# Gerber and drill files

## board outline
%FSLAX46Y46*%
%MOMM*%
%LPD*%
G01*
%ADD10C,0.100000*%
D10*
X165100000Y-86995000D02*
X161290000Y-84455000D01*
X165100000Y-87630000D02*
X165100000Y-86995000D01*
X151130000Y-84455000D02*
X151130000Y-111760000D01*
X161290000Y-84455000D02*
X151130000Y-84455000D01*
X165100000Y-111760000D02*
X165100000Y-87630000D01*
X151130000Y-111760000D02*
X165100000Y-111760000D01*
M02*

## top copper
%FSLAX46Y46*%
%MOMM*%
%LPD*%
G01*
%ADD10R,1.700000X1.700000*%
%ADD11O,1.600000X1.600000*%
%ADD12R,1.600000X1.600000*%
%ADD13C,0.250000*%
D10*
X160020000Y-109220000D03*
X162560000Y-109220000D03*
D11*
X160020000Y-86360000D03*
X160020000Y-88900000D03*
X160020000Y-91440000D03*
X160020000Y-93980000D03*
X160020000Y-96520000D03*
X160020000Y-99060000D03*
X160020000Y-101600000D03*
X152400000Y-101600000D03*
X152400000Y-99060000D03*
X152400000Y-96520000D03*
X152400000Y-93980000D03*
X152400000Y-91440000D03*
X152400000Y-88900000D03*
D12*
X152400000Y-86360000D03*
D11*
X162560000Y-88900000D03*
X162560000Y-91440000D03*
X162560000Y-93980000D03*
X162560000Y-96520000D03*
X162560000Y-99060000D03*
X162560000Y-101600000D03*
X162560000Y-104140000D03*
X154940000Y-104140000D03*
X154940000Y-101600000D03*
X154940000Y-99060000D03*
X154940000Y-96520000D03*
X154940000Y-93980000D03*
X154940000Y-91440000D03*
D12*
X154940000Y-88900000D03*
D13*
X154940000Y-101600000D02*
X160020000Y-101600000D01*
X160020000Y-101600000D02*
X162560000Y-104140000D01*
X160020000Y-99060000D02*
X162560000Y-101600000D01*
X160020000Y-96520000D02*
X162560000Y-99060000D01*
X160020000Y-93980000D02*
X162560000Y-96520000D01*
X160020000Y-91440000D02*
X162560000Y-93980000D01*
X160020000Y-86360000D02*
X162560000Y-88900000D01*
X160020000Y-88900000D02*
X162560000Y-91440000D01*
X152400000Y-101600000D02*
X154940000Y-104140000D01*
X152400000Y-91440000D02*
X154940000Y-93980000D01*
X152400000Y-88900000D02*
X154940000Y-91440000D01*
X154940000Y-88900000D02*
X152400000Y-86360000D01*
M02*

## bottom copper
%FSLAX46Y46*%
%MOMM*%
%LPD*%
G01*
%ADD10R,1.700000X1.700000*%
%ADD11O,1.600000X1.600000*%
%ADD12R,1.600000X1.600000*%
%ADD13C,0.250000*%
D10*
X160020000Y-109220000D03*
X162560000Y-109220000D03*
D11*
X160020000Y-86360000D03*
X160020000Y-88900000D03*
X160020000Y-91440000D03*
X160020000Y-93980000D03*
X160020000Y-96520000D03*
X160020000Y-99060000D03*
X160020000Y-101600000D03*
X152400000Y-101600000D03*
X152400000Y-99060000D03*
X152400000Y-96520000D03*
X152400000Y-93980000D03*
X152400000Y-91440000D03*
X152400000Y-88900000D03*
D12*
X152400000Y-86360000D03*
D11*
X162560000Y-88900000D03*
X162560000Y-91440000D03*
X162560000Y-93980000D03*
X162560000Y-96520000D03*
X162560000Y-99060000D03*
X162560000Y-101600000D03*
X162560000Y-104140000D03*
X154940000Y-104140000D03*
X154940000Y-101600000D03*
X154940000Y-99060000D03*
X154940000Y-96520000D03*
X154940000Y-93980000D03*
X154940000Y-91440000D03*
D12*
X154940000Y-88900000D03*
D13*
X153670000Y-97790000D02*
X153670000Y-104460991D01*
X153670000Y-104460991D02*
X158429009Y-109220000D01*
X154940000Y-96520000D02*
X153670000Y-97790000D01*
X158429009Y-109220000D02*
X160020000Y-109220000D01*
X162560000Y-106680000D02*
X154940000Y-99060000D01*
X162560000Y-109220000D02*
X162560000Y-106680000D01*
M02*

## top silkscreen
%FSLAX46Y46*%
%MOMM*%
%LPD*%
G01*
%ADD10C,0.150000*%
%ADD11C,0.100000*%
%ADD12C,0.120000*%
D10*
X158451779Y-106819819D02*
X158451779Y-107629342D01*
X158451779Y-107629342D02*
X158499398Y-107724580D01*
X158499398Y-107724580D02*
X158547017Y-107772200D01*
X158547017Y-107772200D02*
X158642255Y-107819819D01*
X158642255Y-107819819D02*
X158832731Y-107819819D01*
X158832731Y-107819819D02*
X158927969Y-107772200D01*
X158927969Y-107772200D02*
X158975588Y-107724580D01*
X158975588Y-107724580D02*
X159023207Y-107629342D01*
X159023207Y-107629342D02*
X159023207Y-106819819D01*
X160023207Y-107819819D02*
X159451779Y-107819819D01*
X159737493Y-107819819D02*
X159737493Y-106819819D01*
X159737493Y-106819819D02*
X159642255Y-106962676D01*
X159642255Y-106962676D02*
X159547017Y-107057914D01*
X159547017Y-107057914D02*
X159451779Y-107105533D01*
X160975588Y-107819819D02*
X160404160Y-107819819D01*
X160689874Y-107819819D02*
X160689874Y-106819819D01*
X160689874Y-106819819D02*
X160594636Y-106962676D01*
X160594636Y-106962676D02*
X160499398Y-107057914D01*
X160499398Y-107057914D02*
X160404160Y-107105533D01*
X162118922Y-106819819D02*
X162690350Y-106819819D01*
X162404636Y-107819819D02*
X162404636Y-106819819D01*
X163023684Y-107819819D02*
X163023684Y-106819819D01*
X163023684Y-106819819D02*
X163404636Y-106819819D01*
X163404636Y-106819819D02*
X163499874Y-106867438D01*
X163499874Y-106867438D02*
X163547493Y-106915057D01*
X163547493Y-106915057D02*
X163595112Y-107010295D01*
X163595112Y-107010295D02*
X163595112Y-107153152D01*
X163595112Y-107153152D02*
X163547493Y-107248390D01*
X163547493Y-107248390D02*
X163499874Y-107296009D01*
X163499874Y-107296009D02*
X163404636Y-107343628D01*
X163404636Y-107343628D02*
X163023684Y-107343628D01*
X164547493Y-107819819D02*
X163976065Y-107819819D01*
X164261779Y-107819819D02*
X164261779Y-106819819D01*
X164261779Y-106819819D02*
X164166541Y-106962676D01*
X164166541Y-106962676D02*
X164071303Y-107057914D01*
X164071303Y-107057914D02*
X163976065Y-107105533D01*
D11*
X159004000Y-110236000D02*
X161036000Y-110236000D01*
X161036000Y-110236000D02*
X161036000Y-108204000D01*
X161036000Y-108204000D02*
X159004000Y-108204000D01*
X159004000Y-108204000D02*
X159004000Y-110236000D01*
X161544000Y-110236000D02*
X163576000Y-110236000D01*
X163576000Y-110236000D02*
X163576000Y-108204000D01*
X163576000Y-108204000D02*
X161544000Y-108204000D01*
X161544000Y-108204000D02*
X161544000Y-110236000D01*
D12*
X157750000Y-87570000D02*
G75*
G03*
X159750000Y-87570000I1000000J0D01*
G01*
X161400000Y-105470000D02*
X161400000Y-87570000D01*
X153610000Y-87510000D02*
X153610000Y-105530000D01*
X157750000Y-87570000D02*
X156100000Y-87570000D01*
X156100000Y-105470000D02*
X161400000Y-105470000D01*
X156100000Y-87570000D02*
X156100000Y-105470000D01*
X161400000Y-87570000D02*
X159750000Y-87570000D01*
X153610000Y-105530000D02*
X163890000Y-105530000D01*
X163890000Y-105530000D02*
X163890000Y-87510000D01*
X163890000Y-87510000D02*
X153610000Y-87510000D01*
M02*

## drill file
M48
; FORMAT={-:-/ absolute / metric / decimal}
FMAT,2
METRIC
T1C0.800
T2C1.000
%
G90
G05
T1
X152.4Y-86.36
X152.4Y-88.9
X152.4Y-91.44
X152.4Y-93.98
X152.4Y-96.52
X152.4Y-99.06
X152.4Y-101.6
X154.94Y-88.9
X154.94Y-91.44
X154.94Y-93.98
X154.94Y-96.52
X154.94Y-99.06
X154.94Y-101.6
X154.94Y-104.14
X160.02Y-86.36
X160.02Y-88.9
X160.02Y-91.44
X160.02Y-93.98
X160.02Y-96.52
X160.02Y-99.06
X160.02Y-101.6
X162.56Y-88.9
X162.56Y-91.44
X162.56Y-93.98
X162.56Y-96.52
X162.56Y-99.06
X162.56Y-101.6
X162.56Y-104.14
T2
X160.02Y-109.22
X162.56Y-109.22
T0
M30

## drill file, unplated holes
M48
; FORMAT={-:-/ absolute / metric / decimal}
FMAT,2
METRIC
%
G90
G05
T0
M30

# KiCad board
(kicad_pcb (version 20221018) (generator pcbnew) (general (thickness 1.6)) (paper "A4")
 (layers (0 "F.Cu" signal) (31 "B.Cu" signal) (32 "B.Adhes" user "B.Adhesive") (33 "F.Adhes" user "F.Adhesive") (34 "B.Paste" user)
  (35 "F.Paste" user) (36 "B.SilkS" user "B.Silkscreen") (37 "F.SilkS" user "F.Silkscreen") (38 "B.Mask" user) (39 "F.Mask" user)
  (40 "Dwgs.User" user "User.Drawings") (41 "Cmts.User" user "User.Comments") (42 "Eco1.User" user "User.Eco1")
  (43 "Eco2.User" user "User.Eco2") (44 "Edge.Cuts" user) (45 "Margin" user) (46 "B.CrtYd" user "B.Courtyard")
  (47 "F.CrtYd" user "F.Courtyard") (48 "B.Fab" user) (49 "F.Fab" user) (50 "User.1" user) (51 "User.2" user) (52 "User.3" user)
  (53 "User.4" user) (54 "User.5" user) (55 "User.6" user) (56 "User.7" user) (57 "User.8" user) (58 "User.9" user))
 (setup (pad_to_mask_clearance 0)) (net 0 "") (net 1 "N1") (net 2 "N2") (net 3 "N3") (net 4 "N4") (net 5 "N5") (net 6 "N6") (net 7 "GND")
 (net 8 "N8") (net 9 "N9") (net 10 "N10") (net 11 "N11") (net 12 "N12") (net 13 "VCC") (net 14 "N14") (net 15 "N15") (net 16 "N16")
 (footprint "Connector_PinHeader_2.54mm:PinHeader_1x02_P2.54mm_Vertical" (layer "F.Cu") (at 160.02 109.22 90)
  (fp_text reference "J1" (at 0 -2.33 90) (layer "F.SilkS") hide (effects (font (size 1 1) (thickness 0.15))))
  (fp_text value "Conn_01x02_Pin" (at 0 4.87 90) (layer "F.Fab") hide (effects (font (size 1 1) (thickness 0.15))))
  (fp_rect (start -1.016 -1.016) (end 1.016 1.016) (stroke (width 0.1) (type default)) (fill none) (layer "F.SilkS"))
  (fp_rect (start -1.016 1.524) (end 1.016 3.556) (stroke (width 0.1) (type default)) (fill none) (layer "F.SilkS"))
  (pad "1" thru_hole rect (at 0 0 90) (size 1.7 1.7) (drill 1) (layers "*.Cu" "*.Mask") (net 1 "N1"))
  (pad "2" thru_hole rect (at 0 2.54 90) (size 1.7 1.7) (drill 1) (layers "*.Cu" "*.Mask") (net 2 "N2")))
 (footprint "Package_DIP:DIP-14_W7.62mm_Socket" (layer "F.Cu") (at 154.94 88.9)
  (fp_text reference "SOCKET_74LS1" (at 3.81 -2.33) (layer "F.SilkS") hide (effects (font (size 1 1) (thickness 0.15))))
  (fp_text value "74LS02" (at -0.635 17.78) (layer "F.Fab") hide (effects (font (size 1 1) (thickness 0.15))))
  (fp_line (start -1.33 -1.39) (end -1.33 16.63) (stroke (width 0.12) (type solid)) (layer "F.SilkS"))
  (fp_line (start -1.33 16.63) (end 8.95 16.63) (stroke (width 0.12) (type solid)) (layer "F.SilkS"))
  (fp_line (start 1.16 -1.33) (end 1.16 16.57) (stroke (width 0.12) (type solid)) (layer "F.SilkS"))
  (fp_line (start 1.16 16.57) (end 6.46 16.57) (stroke (width 0.12) (type solid)) (layer "F.SilkS"))
  (fp_line (start 2.81 -1.33) (end 1.16 -1.33) (stroke (width 0.12) (type solid)) (layer "F.SilkS"))
  (fp_line (start 6.46 -1.33) (end 4.81 -1.33) (stroke (width 0.12) (type solid)) (layer "F.SilkS"))
  (fp_line (start 6.46 16.57) (end 6.46 -1.33) (stroke (width 0.12) (type solid)) (layer "F.SilkS"))
  (fp_line (start 8.95 -1.39) (end -1.33 -1.39) (stroke (width 0.12) (type solid)) (layer "F.SilkS"))
  (fp_line (start 8.95 16.63) (end 8.95 -1.39) (stroke (width 0.12) (type solid)) (layer "F.SilkS"))
  (fp_arc (start 4.81 -1.33) (mid 3.81 -0.33) (end 2.81 -1.33) (stroke (width 0.12) (type solid)) (layer "F.SilkS"))
  (pad "1" thru_hole rect (at 0 0) (size 1.6 1.6) (drill 0.8) (layers "*.Cu" "*.Mask") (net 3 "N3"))
  (pad "2" thru_hole oval (at 0 2.54) (size 1.6 1.6) (drill 0.8) (layers "*.Cu" "*.Mask") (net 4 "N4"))
  (pad "3" thru_hole oval (at 0 5.08) (size 1.6 1.6) (drill 0.8) (layers "*.Cu" "*.Mask") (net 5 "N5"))
  (pad "4" thru_hole oval (at 0 7.62) (size 1.6 1.6) (drill 0.8) (layers "*.Cu" "*.Mask") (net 1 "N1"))
  (pad "5" thru_hole oval (at 0 10.16) (size 1.6 1.6) (drill 0.8) (layers "*.Cu" "*.Mask") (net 2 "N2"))
  (pad "6" thru_hole oval (at 0 12.7) (size 1.6 1.6) (drill 0.8) (layers "*.Cu" "*.Mask") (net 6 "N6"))
  (pad "7" thru_hole oval (at 0 15.24) (size 1.6 1.6) (drill 0.8) (layers "*.Cu" "*.Mask") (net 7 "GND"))
  (pad "8" thru_hole oval (at 7.62 15.24) (size 1.6 1.6) (drill 0.8) (layers "*.Cu" "*.Mask") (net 6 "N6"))
  (pad "9" thru_hole oval (at 7.62 12.7) (size 1.6 1.6) (drill 0.8) (layers "*.Cu" "*.Mask") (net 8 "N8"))
  (pad "10" thru_hole oval (at 7.62 10.16) (size 1.6 1.6) (drill 0.8) (layers "*.Cu" "*.Mask") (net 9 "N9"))
  (pad "11" thru_hole oval (at 7.62 7.62) (size 1.6 1.6) (drill 0.8) (layers "*.Cu" "*.Mask") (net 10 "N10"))
  (pad "12" thru_hole oval (at 7.62 5.08) (size 1.6 1.6) (drill 0.8) (layers "*.Cu" "*.Mask") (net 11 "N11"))
  (pad "13" thru_hole oval (at 7.62 2.54) (size 1.6 1.6) (drill 0.8) (layers "*.Cu" "*.Mask") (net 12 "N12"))
  (pad "14" thru_hole oval (at 7.62 0) (size 1.6 1.6) (drill 0.8) (layers "*.Cu" "*.Mask") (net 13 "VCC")))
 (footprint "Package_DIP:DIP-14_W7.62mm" (layer "F.Cu") (at 152.4 86.36)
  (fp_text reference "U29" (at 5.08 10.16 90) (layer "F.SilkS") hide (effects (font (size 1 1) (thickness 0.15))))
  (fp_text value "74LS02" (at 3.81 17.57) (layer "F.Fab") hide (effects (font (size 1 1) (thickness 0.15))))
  (pad "1" thru_hole rect (at 0 0) (size 1.6 1.6) (drill 0.8) (layers "*.Cu" "*.Mask") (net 3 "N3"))
  (pad "2" thru_hole oval (at 0 2.54) (size 1.6 1.6) (drill 0.8) (layers "*.Cu" "*.Mask") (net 4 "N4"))
  (pad "3" thru_hole oval (at 0 5.08) (size 1.6 1.6) (drill 0.8) (layers "*.Cu" "*.Mask") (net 5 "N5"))
  (pad "4" thru_hole oval (at 0 7.62) (size 1.6 1.6) (drill 0.8) (layers "*.Cu" "*.Mask") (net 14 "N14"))
  (pad "5" thru_hole oval (at 0 10.16) (size 1.6 1.6) (drill 0.8) (layers "*.Cu" "*.Mask") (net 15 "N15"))
  (pad "6" thru_hole oval (at 0 12.7) (size 1.6 1.6) (drill 0.8) (layers "*.Cu" "*.Mask") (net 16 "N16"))
  (pad "7" thru_hole oval (at 0 15.24) (size 1.6 1.6) (drill 0.8) (layers "*.Cu" "*.Mask") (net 7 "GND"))
  (pad "8" thru_hole oval (at 7.62 15.24) (size 1.6 1.6) (drill 0.8) (layers "*.Cu" "*.Mask") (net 6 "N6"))
  (pad "9" thru_hole oval (at 7.62 12.7) (size 1.6 1.6) (drill 0.8) (layers "*.Cu" "*.Mask") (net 8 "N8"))
  (pad "10" thru_hole oval (at 7.62 10.16) (size 1.6 1.6) (drill 0.8) (layers "*.Cu" "*.Mask") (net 9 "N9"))
  (pad "11" thru_hole oval (at 7.62 7.62) (size 1.6 1.6) (drill 0.8) (layers "*.Cu" "*.Mask") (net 10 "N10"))
  (pad "12" thru_hole oval (at 7.62 5.08) (size 1.6 1.6) (drill 0.8) (layers "*.Cu" "*.Mask") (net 11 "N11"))
  (pad "13" thru_hole oval (at 7.62 2.54) (size 1.6 1.6) (drill 0.8) (layers "*.Cu" "*.Mask") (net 12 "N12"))
  (pad "14" thru_hole oval (at 7.62 0) (size 1.6 1.6) (drill 0.8) (layers "*.Cu" "*.Mask") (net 13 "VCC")))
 (gr_line (start 165.1 87.63) (end 165.1 86.995) (stroke (width 0.1) (type default)) (layer "Edge.Cuts"))
 (gr_line (start 151.13 84.455) (end 151.13 111.76) (stroke (width 0.1) (type default)) (layer "Edge.Cuts"))
 (gr_line (start 161.29 84.455) (end 151.13 84.455) (stroke (width 0.1) (type default)) (layer "Edge.Cuts"))
 (gr_line (start 165.1 86.995) (end 161.29 84.455) (stroke (width 0.1) (type default)) (layer "Edge.Cuts"))
 (gr_line (start 165.1 111.76) (end 165.1 87.63) (stroke (width 0.1) (type default)) (layer "Edge.Cuts"))
 (gr_line (start 151.13 111.76) (end 165.1 111.76) (stroke (width 0.1) (type default)) (layer "Edge.Cuts"))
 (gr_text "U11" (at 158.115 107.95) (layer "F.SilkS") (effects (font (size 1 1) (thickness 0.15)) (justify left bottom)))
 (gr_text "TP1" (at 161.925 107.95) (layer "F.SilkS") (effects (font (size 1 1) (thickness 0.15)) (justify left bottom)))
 (segment (start 158.429009 109.22) (end 160.02 109.22) (width 0.25) (layer "B.Cu") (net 1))
 (segment (start 153.67 97.79) (end 153.67 104.460991) (width 0.25) (layer "B.Cu") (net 1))
 (segment (start 154.94 96.52) (end 153.67 97.79) (width 0.25) (layer "B.Cu") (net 1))
 (segment (start 153.67 104.460991) (end 158.429009 109.22) (width 0.25) (layer "B.Cu") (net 1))
 (segment (start 162.56 109.22) (end 162.56 106.68) (width 0.25) (layer "B.Cu") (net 2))
 (segment (start 162.56 106.68) (end 154.94 99.06) (width 0.25) (layer "B.Cu") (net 2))
 (segment (start 154.94 88.9) (end 152.4 86.36) (width 0.25) (layer "F.Cu") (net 3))
 (segment (start 152.4 88.9) (end 154.94 91.44) (width 0.25) (layer "F.Cu") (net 4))
 (segment (start 152.4 91.44) (end 154.94 93.98) (width 0.25) (layer "F.Cu") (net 5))
 (segment (start 160.02 101.6) (end 162.56 104.14) (width 0.25) (layer "F.Cu") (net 6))
 (segment (start 154.94 101.6) (end 160.02 101.6) (width 0.25) (layer "F.Cu") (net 6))
 (segment (start 152.4 101.6) (end 154.94 104.14) (width 0.25) (layer "F.Cu") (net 7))
 (segment (start 160.02 99.06) (end 162.56 101.6) (width 0.25) (layer "F.Cu") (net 8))
 (segment (start 160.02 96.52) (end 162.56 99.06) (width 0.25) (layer "F.Cu") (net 9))
 (segment (start 160.02 93.98) (end 162.56 96.52) (width 0.25) (layer "F.Cu") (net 10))
 (segment (start 160.02 91.44) (end 162.56 93.98) (width 0.25) (layer "F.Cu") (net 11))
 (segment (start 160.02 88.9) (end 162.56 91.44) (width 0.25) (layer "F.Cu") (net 12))
 (segment (start 160.02 86.36) (end 162.56 88.9) (width 0.25) (layer "F.Cu") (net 13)))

